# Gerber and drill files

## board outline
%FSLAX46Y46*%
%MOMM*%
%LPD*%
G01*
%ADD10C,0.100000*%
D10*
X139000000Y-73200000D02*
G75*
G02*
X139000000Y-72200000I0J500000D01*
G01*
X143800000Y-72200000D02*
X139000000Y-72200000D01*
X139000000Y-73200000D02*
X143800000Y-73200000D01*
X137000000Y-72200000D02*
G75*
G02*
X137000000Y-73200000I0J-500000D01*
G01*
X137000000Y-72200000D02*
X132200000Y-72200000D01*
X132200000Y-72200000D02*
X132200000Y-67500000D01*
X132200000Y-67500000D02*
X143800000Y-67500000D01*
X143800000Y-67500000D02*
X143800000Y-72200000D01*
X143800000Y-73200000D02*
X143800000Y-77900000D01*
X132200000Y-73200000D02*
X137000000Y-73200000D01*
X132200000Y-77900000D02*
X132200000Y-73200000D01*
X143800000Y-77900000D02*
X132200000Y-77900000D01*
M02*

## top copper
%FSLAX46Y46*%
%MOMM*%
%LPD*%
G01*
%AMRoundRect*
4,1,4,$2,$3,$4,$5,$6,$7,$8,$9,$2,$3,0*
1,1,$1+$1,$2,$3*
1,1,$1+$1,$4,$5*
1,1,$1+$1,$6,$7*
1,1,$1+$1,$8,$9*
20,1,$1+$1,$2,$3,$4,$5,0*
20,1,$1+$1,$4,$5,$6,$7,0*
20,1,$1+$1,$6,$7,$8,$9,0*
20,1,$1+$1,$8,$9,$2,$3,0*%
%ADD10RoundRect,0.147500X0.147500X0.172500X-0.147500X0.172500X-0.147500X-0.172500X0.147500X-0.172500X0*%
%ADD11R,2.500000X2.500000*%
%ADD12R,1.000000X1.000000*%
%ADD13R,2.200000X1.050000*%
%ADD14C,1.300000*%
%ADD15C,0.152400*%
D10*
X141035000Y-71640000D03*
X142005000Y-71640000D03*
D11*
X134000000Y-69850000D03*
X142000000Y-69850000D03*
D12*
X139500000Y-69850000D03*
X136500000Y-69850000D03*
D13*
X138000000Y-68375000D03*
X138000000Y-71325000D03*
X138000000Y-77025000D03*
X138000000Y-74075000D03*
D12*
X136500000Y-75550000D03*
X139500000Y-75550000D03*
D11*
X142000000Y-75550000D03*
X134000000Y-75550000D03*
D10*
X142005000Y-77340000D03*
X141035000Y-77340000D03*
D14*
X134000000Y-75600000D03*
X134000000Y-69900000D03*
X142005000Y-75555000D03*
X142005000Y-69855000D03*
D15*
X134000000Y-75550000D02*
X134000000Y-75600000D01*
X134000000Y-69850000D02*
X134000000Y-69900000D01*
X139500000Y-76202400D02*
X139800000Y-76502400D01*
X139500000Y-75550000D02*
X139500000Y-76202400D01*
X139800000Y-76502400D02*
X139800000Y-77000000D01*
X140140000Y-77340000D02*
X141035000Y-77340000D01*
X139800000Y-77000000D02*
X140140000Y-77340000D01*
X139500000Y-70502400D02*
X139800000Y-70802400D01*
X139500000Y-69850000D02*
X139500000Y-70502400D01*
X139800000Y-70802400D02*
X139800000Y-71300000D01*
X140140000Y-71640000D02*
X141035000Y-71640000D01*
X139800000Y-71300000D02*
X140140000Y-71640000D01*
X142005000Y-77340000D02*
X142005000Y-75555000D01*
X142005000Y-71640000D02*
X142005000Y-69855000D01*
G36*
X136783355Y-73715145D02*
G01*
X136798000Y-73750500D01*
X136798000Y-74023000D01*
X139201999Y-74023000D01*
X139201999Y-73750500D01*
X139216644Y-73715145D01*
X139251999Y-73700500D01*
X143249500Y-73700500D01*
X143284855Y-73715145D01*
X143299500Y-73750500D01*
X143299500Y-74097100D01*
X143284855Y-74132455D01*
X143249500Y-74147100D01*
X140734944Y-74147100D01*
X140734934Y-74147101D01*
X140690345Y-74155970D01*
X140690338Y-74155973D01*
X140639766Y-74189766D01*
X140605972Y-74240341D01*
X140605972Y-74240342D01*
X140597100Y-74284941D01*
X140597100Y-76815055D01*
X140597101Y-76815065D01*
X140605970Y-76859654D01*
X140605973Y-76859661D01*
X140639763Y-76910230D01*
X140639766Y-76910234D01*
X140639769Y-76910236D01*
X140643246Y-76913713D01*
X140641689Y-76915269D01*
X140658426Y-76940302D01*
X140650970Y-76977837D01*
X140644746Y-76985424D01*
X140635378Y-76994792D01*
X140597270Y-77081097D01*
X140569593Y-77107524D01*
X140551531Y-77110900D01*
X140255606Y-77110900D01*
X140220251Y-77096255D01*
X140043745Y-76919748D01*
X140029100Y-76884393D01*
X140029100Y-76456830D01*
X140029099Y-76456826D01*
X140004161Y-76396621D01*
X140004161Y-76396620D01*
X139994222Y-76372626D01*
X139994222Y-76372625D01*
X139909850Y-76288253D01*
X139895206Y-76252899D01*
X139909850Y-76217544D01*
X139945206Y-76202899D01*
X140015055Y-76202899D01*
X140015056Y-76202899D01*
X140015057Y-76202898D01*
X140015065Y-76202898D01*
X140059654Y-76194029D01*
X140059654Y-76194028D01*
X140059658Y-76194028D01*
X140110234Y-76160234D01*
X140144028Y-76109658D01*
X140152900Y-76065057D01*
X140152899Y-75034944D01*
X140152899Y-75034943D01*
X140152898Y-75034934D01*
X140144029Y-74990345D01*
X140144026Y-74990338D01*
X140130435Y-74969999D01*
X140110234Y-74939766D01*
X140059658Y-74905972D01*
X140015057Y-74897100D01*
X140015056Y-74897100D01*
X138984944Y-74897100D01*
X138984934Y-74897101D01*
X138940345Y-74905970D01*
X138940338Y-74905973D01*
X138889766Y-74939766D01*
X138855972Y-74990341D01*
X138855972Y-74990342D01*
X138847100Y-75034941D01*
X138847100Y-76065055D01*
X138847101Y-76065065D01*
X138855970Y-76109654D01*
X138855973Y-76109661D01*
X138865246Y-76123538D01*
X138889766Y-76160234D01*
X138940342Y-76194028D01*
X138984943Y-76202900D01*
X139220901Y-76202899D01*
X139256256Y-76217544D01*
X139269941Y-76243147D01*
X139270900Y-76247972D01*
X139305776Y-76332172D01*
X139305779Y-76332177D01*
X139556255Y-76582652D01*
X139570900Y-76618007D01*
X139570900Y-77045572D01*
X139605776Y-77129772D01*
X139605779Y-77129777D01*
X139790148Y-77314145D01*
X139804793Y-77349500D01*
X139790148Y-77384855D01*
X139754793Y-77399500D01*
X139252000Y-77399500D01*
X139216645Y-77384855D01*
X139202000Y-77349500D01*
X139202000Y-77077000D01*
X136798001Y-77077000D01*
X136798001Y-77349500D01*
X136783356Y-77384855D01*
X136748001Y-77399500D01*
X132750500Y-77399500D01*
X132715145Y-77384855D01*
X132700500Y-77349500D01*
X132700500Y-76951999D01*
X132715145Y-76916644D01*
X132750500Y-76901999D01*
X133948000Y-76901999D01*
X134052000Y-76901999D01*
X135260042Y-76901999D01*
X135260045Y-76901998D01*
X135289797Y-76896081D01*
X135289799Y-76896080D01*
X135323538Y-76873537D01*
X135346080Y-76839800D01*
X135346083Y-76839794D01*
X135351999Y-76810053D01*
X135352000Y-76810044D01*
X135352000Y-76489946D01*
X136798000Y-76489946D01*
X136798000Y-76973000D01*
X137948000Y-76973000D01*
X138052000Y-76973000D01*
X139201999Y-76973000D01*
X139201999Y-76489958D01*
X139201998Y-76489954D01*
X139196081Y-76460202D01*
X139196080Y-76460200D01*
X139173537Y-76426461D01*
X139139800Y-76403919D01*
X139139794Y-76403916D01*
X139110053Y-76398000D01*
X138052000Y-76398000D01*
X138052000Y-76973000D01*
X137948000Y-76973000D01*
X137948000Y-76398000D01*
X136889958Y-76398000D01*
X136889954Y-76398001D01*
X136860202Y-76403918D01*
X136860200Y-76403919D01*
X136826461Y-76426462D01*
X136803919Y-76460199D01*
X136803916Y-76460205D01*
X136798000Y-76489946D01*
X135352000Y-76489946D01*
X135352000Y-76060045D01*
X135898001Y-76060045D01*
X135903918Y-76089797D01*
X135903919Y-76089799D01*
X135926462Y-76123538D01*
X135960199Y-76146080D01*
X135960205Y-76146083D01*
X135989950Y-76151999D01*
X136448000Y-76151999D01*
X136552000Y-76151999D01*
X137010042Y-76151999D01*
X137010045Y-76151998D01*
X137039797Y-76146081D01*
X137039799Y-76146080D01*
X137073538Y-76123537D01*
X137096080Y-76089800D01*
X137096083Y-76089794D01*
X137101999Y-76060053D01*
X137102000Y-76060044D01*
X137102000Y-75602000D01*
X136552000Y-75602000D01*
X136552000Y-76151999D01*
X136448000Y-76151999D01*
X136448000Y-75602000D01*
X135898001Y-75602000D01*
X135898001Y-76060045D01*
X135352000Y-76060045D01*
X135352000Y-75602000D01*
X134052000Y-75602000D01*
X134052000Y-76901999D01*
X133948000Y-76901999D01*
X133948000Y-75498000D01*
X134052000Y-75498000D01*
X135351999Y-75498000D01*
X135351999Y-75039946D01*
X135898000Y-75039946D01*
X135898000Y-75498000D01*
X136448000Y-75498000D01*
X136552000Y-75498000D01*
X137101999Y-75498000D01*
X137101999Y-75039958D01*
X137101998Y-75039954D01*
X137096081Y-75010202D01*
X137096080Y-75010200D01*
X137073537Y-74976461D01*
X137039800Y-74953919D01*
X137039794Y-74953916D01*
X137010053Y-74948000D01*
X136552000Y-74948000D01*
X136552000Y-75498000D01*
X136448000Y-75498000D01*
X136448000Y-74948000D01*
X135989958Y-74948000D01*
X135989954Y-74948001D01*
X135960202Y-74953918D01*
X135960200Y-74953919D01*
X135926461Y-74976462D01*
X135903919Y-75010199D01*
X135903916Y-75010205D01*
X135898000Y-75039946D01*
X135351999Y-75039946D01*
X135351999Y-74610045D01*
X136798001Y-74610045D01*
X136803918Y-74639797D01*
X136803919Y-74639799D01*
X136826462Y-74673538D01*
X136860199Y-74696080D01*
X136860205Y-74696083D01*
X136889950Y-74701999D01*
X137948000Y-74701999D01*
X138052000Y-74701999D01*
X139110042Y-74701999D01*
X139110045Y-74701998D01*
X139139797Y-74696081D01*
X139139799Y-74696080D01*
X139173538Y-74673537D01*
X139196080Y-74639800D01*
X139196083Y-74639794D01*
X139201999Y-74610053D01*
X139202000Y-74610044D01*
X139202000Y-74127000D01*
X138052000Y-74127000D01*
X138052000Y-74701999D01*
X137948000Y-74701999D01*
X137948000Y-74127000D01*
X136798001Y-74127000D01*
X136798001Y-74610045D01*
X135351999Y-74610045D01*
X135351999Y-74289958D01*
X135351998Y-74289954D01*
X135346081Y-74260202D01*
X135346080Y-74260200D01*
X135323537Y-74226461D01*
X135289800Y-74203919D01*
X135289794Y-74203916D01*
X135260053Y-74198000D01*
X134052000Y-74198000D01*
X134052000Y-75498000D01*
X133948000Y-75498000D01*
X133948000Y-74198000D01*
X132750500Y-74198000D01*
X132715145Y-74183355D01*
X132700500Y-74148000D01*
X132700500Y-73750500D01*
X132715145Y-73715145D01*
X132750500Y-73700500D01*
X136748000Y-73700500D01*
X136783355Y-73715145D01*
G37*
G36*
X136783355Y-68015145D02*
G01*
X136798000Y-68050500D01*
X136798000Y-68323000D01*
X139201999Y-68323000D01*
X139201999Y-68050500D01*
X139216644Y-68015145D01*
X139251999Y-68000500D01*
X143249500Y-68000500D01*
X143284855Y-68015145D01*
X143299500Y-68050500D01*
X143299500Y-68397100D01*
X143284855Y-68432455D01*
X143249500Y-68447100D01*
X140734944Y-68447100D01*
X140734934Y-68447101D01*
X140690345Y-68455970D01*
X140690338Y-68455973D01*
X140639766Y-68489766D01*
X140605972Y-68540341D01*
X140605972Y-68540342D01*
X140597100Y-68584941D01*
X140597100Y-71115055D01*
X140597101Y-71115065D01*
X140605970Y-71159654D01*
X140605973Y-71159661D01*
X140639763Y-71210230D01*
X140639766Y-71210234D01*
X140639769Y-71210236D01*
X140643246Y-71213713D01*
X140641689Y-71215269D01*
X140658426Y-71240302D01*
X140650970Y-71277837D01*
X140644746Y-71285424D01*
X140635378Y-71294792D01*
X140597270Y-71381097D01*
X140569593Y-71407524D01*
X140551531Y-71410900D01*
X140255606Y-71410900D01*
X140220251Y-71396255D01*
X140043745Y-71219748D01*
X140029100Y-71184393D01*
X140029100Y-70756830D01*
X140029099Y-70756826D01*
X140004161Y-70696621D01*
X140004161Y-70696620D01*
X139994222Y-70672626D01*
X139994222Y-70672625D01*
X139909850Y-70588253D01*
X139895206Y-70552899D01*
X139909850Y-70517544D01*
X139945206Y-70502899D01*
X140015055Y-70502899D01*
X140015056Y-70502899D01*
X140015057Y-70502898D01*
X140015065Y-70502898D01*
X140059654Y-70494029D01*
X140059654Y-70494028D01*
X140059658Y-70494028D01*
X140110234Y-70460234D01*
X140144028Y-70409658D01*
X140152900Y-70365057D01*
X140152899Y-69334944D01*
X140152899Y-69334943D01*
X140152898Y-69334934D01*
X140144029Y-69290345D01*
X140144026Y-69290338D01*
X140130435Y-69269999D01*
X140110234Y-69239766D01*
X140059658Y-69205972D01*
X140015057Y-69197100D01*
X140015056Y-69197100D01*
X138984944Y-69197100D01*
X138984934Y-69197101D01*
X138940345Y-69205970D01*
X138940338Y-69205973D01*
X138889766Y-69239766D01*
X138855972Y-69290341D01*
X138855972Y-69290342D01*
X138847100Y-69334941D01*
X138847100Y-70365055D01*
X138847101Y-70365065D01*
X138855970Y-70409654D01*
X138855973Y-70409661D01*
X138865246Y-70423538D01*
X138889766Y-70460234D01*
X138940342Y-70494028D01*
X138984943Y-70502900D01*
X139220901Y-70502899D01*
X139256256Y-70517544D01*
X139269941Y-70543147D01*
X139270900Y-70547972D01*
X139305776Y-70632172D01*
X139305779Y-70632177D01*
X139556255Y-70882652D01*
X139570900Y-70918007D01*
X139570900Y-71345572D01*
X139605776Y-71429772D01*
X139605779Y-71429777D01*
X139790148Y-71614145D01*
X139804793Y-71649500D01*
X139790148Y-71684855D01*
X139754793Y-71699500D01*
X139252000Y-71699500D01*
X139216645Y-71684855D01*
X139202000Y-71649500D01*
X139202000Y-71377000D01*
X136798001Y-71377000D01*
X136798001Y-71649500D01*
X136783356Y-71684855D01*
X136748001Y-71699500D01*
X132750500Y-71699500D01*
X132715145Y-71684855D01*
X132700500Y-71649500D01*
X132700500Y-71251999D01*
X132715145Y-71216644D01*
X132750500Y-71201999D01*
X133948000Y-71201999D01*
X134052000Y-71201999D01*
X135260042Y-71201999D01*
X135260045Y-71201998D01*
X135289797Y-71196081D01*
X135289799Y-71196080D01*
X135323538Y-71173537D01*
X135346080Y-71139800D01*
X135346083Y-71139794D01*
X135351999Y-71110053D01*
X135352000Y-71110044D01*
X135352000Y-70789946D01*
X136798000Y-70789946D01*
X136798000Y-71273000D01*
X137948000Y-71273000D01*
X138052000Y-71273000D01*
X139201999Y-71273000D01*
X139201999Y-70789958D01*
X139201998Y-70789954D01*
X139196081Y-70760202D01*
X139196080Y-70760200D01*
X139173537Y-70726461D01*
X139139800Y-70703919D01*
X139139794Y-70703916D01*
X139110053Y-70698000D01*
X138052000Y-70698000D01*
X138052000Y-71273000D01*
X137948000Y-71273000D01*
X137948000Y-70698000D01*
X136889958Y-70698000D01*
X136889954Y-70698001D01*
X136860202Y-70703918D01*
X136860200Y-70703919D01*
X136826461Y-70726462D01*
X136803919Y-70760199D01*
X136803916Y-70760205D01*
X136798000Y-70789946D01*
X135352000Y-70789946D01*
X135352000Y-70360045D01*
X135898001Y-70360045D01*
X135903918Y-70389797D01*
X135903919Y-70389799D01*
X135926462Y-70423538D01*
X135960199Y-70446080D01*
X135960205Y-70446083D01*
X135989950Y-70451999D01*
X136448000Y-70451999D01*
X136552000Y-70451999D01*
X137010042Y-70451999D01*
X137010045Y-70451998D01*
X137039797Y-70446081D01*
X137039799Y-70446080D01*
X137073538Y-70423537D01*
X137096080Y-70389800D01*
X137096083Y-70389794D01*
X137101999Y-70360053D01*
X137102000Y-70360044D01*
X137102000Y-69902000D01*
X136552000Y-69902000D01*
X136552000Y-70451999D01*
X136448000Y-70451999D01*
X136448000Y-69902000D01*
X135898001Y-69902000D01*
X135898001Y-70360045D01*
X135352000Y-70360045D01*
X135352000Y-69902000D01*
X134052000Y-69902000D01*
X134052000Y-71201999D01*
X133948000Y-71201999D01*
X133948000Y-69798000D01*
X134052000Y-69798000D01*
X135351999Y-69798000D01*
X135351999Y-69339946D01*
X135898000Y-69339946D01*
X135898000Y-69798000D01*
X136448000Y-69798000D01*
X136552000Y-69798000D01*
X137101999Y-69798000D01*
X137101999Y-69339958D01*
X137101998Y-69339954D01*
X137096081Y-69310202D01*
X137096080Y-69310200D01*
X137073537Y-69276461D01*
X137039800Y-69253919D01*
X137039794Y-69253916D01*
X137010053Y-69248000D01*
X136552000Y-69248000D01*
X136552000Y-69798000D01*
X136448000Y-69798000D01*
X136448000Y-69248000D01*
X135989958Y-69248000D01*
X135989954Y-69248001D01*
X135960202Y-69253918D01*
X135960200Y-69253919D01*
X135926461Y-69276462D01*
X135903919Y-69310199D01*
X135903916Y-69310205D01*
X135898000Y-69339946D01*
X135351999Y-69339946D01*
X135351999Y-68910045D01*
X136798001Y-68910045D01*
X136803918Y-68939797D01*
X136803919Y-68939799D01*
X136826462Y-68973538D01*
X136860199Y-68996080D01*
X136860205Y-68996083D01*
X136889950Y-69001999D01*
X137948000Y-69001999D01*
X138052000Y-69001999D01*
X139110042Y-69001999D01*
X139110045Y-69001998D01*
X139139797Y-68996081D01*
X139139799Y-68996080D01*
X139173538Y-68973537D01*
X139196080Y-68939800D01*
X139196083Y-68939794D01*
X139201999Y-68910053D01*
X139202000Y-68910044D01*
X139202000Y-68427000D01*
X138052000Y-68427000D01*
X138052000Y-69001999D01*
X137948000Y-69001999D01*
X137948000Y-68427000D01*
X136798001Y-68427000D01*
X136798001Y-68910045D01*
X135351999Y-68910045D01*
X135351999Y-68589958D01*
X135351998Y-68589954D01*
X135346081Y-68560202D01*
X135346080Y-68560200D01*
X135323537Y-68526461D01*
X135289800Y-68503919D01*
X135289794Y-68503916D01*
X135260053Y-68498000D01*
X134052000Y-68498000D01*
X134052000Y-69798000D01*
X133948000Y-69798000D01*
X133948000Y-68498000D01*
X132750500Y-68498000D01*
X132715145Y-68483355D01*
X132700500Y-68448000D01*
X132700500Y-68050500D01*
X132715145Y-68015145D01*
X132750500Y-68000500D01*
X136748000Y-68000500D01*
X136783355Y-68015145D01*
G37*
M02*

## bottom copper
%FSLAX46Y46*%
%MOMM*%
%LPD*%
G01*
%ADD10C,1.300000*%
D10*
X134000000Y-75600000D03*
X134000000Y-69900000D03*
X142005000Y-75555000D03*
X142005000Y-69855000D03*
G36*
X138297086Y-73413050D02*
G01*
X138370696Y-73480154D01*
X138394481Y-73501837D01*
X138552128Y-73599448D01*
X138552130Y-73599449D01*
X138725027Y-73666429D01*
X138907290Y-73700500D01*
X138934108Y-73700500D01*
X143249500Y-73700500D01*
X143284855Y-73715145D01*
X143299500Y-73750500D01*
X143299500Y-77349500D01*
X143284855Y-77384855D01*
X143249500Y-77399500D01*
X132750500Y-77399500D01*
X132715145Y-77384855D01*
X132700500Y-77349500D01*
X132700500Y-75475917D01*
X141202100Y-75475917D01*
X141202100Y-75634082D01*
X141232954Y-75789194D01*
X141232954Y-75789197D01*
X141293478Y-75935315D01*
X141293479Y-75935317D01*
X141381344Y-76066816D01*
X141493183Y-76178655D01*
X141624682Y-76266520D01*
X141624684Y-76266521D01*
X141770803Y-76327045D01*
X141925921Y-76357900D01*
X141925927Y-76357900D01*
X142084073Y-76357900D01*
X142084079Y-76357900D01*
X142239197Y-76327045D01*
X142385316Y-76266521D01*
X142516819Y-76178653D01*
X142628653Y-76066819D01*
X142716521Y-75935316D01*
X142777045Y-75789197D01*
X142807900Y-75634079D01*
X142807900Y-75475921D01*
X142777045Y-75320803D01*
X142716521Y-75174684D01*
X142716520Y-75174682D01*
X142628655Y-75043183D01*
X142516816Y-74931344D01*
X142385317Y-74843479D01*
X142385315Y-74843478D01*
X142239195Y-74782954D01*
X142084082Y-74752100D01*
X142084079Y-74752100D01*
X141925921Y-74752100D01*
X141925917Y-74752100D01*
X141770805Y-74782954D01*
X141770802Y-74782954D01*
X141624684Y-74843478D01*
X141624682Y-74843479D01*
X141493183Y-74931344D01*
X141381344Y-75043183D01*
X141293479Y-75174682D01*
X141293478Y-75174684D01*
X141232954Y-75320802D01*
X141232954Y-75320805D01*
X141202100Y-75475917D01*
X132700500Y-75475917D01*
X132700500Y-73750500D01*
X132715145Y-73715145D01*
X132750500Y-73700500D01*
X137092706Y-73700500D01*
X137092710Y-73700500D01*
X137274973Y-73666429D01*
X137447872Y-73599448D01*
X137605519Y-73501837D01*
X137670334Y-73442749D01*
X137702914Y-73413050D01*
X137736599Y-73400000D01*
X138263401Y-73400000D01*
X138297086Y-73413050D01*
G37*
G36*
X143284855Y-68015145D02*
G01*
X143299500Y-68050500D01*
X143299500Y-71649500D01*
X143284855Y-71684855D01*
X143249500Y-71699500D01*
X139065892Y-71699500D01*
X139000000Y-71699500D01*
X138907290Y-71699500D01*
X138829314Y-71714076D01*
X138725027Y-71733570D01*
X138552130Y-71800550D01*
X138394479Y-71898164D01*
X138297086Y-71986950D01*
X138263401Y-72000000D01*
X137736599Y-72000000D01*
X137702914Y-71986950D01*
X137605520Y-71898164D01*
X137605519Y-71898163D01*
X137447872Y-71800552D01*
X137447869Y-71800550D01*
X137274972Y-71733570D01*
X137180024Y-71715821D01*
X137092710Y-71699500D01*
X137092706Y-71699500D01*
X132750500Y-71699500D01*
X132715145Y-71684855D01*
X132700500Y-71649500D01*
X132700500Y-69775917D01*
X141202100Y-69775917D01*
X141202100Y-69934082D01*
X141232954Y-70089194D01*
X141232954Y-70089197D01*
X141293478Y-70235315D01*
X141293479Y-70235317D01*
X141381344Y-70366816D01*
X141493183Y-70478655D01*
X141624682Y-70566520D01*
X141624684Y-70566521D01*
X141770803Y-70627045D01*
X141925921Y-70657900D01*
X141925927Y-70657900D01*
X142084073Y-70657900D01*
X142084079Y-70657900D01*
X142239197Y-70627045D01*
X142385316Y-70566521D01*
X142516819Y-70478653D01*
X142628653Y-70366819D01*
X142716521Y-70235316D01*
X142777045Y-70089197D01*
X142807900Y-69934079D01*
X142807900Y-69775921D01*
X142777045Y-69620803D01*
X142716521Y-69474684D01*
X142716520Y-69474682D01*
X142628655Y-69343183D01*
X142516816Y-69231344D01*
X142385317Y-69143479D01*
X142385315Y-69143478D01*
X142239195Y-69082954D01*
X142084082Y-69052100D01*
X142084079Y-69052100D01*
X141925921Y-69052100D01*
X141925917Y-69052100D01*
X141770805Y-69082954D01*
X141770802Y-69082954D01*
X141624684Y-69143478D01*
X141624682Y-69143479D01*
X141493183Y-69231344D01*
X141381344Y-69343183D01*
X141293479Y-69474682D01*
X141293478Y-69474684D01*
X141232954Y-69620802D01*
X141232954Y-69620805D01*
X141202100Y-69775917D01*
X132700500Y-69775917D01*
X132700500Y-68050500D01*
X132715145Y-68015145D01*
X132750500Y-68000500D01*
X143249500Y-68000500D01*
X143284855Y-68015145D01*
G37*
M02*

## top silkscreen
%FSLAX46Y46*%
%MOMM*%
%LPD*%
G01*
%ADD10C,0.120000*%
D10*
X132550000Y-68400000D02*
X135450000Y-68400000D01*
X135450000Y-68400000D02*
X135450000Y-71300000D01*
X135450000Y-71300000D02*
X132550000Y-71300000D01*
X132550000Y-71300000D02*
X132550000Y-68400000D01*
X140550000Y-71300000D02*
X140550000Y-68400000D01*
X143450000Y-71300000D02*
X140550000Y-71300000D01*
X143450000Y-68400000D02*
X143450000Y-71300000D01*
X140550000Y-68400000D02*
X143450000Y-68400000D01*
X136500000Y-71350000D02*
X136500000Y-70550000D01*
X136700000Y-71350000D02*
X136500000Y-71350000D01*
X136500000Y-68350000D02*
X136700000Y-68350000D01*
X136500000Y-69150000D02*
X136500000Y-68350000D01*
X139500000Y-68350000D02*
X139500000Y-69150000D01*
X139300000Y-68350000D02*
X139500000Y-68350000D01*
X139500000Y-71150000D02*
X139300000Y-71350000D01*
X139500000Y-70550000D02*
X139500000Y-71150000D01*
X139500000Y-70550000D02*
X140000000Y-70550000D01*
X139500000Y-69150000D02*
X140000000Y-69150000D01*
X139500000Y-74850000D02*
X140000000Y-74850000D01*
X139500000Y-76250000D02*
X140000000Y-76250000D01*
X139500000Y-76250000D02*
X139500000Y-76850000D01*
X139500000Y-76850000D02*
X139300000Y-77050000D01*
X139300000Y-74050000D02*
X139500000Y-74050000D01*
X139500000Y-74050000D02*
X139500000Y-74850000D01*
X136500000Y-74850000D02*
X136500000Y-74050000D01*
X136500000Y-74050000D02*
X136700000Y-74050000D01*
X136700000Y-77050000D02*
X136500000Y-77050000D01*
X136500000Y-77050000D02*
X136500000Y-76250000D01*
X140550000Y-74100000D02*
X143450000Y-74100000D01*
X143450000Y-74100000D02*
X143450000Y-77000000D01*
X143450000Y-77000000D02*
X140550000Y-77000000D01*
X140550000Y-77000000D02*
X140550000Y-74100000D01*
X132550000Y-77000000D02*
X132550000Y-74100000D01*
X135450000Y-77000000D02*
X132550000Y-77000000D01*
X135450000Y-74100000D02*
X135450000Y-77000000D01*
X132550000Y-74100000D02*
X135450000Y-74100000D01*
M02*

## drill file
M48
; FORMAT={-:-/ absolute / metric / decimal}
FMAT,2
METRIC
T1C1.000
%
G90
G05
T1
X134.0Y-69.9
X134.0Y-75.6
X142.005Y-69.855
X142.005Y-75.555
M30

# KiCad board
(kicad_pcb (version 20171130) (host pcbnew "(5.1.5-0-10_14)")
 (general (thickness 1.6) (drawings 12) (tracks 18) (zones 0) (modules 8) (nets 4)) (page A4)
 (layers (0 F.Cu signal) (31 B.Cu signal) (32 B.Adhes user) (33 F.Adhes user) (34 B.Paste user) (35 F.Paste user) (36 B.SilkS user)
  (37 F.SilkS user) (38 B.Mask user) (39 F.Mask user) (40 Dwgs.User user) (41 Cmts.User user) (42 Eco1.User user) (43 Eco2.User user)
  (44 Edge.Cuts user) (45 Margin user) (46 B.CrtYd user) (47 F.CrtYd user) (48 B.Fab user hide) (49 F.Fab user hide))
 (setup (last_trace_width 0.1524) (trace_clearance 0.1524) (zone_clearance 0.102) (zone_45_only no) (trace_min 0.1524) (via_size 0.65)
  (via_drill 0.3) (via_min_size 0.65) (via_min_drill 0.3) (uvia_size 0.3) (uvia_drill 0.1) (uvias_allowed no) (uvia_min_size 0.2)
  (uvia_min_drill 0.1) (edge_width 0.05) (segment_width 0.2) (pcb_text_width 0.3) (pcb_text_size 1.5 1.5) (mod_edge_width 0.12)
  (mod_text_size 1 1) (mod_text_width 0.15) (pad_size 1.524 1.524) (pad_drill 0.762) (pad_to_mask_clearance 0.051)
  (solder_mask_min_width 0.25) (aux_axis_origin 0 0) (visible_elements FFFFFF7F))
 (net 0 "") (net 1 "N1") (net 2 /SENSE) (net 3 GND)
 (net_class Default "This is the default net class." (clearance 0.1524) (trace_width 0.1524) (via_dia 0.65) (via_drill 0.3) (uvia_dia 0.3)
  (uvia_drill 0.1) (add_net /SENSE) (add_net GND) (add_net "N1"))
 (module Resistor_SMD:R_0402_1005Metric (layer F.Cu) (at 141.52 71.64 180)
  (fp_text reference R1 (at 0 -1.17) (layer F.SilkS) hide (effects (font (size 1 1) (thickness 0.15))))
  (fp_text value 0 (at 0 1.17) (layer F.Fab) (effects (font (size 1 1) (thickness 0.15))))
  (pad 2 smd roundrect (at 0.485 0 180) (size 0.59 0.64) (layers F.Cu F.Paste F.Mask) (roundrect_rratio 0.25) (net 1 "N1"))
  (pad 1 smd roundrect (at -0.485 0 180) (size 0.59 0.64) (layers F.Cu F.Paste F.Mask) (roundrect_rratio 0.25) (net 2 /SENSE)))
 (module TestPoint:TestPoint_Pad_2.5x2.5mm (layer F.Cu) (at 134 69.85)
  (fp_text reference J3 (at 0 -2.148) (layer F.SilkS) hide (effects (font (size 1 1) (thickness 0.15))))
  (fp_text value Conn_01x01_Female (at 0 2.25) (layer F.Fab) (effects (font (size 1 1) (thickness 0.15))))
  (fp_line (start -1.45 -1.45) (end 1.45 -1.45) (layer F.SilkS) (width 0.12))
  (fp_line (start 1.45 -1.45) (end 1.45 1.45) (layer F.SilkS) (width 0.12))
  (fp_line (start 1.45 1.45) (end -1.45 1.45) (layer F.SilkS) (width 0.12))
  (fp_line (start -1.45 1.45) (end -1.45 -1.45) (layer F.SilkS) (width 0.12))
  (pad 1 smd rect (at 0 0) (size 2.5 2.5) (layers F.Cu F.Mask) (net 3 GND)))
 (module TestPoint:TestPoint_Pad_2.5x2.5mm (layer F.Cu) (at 142 69.85)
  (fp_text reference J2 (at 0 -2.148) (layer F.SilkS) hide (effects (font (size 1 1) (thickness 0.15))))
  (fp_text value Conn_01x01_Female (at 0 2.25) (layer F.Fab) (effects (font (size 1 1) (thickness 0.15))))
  (fp_line (start -1.45 1.45) (end -1.45 -1.45) (layer F.SilkS) (width 0.12))
  (fp_line (start 1.45 1.45) (end -1.45 1.45) (layer F.SilkS) (width 0.12))
  (fp_line (start 1.45 -1.45) (end 1.45 1.45) (layer F.SilkS) (width 0.12))
  (fp_line (start -1.45 -1.45) (end 1.45 -1.45) (layer F.SilkS) (width 0.12))
  (pad 1 smd rect (at 0 0) (size 2.5 2.5) (layers F.Cu F.Mask) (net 2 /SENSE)))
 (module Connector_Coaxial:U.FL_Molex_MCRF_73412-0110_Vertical (layer F.Cu) (at 138 69.85 90)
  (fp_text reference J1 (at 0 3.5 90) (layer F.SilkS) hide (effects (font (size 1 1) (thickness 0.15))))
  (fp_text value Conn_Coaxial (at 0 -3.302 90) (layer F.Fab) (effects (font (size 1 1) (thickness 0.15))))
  (fp_line (start -1.5 -1.5) (end -0.7 -1.5) (layer F.SilkS) (width 0.12))
  (fp_line (start -1.5 -1.3) (end -1.5 -1.5) (layer F.SilkS) (width 0.12))
  (fp_line (start 1.5 -1.5) (end 1.5 -1.3) (layer F.SilkS) (width 0.12))
  (fp_line (start 0.7 -1.5) (end 1.5 -1.5) (layer F.SilkS) (width 0.12))
  (fp_line (start 1.5 1.5) (end 0.7 1.5) (layer F.SilkS) (width 0.12))
  (fp_line (start 1.5 1.3) (end 1.5 1.5) (layer F.SilkS) (width 0.12))
  (fp_line (start -1.3 1.5) (end -1.5 1.3) (layer F.SilkS) (width 0.12))
  (fp_line (start -0.7 1.5) (end -1.3 1.5) (layer F.SilkS) (width 0.12))
  (fp_line (start -0.7 1.5) (end -0.7 2) (layer F.SilkS) (width 0.12))
  (fp_line (start 0.7 1.5) (end 0.7 2) (layer F.SilkS) (width 0.12))
  (pad 1 smd rect (at 0 1.5 90) (size 1 1) (layers F.Cu F.Paste F.Mask) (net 1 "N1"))
  (pad 2 smd rect (at 0 -1.5 90) (size 1 1) (layers F.Cu F.Paste F.Mask) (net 3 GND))
  (pad 2 smd rect (at 1.475 0 90) (size 1.05 2.2) (layers F.Cu F.Paste F.Mask) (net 3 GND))
  (pad 2 smd rect (at -1.475 0 90) (size 1.05 2.2) (layers F.Cu F.Paste F.Mask) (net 3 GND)))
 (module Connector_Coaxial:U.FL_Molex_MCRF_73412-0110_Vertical (layer F.Cu) (at 138 75.55 90)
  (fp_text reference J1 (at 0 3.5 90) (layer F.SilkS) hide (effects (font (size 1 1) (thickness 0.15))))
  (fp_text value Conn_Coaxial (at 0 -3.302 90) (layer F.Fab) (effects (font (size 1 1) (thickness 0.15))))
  (fp_line (start 0.7 1.5) (end 0.7 2) (layer F.SilkS) (width 0.12))
  (fp_line (start -0.7 1.5) (end -0.7 2) (layer F.SilkS) (width 0.12))
  (fp_line (start -0.7 1.5) (end -1.3 1.5) (layer F.SilkS) (width 0.12))
  (fp_line (start -1.3 1.5) (end -1.5 1.3) (layer F.SilkS) (width 0.12))
  (fp_line (start 1.5 1.3) (end 1.5 1.5) (layer F.SilkS) (width 0.12))
  (fp_line (start 1.5 1.5) (end 0.7 1.5) (layer F.SilkS) (width 0.12))
  (fp_line (start 0.7 -1.5) (end 1.5 -1.5) (layer F.SilkS) (width 0.12))
  (fp_line (start 1.5 -1.5) (end 1.5 -1.3) (layer F.SilkS) (width 0.12))
  (fp_line (start -1.5 -1.3) (end -1.5 -1.5) (layer F.SilkS) (width 0.12))
  (fp_line (start -1.5 -1.5) (end -0.7 -1.5) (layer F.SilkS) (width 0.12))
  (pad 2 smd rect (at -1.475 0 90) (size 1.05 2.2) (layers F.Cu F.Paste F.Mask) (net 3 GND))
  (pad 2 smd rect (at 1.475 0 90) (size 1.05 2.2) (layers F.Cu F.Paste F.Mask) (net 3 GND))
  (pad 2 smd rect (at 0 -1.5 90) (size 1 1) (layers F.Cu F.Paste F.Mask) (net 3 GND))
  (pad 1 smd rect (at 0 1.5 90) (size 1 1) (layers F.Cu F.Paste F.Mask) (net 1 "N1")))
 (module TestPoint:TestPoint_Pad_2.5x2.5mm (layer F.Cu) (at 142 75.55)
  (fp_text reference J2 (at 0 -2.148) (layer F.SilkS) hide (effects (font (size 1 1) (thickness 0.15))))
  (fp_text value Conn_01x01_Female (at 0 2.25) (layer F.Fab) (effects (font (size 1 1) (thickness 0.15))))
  (fp_line (start -1.45 -1.45) (end 1.45 -1.45) (layer F.SilkS) (width 0.12))
  (fp_line (start 1.45 -1.45) (end 1.45 1.45) (layer F.SilkS) (width 0.12))
  (fp_line (start 1.45 1.45) (end -1.45 1.45) (layer F.SilkS) (width 0.12))
  (fp_line (start -1.45 1.45) (end -1.45 -1.45) (layer F.SilkS) (width 0.12))
  (pad 1 smd rect (at 0 0) (size 2.5 2.5) (layers F.Cu F.Mask) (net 2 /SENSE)))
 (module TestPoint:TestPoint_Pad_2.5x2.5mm (layer F.Cu) (at 134 75.55)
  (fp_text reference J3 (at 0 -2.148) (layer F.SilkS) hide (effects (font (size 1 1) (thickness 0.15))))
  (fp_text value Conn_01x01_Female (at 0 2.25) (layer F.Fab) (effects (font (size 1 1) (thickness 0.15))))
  (fp_line (start -1.45 1.45) (end -1.45 -1.45) (layer F.SilkS) (width 0.12))
  (fp_line (start 1.45 1.45) (end -1.45 1.45) (layer F.SilkS) (width 0.12))
  (fp_line (start 1.45 -1.45) (end 1.45 1.45) (layer F.SilkS) (width 0.12))
  (fp_line (start -1.45 -1.45) (end 1.45 -1.45) (layer F.SilkS) (width 0.12))
  (pad 1 smd rect (at 0 0) (size 2.5 2.5) (layers F.Cu F.Mask) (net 3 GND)))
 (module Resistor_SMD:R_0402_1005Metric (layer F.Cu) (at 141.52 77.34 180)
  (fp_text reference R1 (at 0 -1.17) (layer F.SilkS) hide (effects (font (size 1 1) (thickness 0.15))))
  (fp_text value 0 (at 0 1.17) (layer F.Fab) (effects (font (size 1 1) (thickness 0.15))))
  (pad 1 smd roundrect (at -0.485 0 180) (size 0.59 0.64) (layers F.Cu F.Paste F.Mask) (roundrect_rratio 0.25) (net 2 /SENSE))
  (pad 2 smd roundrect (at 0.485 0 180) (size 0.59 0.64) (layers F.Cu F.Paste F.Mask) (roundrect_rratio 0.25) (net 1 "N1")))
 (gr_arc (start 139 72.7) (end 139 72.2) (angle -180) (layer Edge.Cuts) (width 0.1))
 (gr_line (start 143.8 72.2) (end 139 72.2) (layer Edge.Cuts) (width 0.1))
 (gr_line (start 139 73.2) (end 143.8 73.2) (layer Edge.Cuts) (width 0.1))
 (gr_arc (start 137 72.7) (end 137 73.2) (angle -180) (layer Edge.Cuts) (width 0.1))
 (gr_line (start 137 72.2) (end 132.2 72.2) (layer Edge.Cuts) (width 0.1))
 (gr_line (start 132.2 72.2) (end 132.2 67.5) (layer Edge.Cuts) (width 0.1))
 (gr_line (start 132.2 67.5) (end 143.8 67.5) (layer Edge.Cuts) (width 0.1))
 (gr_line (start 143.8 67.5) (end 143.8 72.2) (layer Edge.Cuts) (width 0.1))
 (gr_line (start 143.8 73.2) (end 143.8 77.9) (layer Edge.Cuts) (width 0.1))
 (gr_line (start 132.2 73.2) (end 137 73.2) (layer Edge.Cuts) (width 0.1))
 (gr_line (start 132.2 77.9) (end 132.2 73.2) (layer Edge.Cuts) (width 0.1))
 (gr_line (start 143.8 77.9) (end 132.2 77.9) (layer Edge.Cuts) (width 0.1))
 (via (at 134 75.6) (size 1.3) (drill 1) (layers F.Cu B.Cu) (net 3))
 (segment (start 134 75.55) (end 134 75.6) (width 0.1524) (layer F.Cu) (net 3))
 (via (at 134 69.9) (size 1.3) (drill 1) (layers F.Cu B.Cu) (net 3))
 (segment (start 134 69.85) (end 134 69.9) (width 0.1524) (layer F.Cu) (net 3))
 (segment (start 139.5 76.2024) (end 139.8 76.5024) (width 0.1524) (layer F.Cu) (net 1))
 (segment (start 139.5 75.55) (end 139.5 76.2024) (width 0.1524) (layer F.Cu) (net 1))
 (segment (start 139.8 76.5024) (end 139.8 77) (width 0.1524) (layer F.Cu) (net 1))
 (segment (start 140.14 77.34) (end 141.035 77.34) (width 0.1524) (layer F.Cu) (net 1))
 (segment (start 139.8 77) (end 140.14 77.34) (width 0.1524) (layer F.Cu) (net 1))
 (segment (start 139.5 70.5024) (end 139.8 70.8024) (width 0.1524) (layer F.Cu) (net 1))
 (segment (start 139.5 69.85) (end 139.5 70.5024) (width 0.1524) (layer F.Cu) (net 1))
 (segment (start 139.8 70.8024) (end 139.8 71.3) (width 0.1524) (layer F.Cu) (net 1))
 (segment (start 140.14 71.64) (end 141.035 71.64) (width 0.1524) (layer F.Cu) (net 1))
 (segment (start 139.8 71.3) (end 140.14 71.64) (width 0.1524) (layer F.Cu) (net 1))
 (segment (start 142.005 77.34) (end 142.005 75.555) (width 0.1524) (layer F.Cu) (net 2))
 (via (at 142.005 75.555) (size 1.3) (drill 1) (layers F.Cu B.Cu) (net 2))
 (segment (start 142.005 71.64) (end 142.005 69.855) (width 0.1524) (layer F.Cu) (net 2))
 (via (at 142.005 69.855) (size 1.3) (drill 1) (layers F.Cu B.Cu) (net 2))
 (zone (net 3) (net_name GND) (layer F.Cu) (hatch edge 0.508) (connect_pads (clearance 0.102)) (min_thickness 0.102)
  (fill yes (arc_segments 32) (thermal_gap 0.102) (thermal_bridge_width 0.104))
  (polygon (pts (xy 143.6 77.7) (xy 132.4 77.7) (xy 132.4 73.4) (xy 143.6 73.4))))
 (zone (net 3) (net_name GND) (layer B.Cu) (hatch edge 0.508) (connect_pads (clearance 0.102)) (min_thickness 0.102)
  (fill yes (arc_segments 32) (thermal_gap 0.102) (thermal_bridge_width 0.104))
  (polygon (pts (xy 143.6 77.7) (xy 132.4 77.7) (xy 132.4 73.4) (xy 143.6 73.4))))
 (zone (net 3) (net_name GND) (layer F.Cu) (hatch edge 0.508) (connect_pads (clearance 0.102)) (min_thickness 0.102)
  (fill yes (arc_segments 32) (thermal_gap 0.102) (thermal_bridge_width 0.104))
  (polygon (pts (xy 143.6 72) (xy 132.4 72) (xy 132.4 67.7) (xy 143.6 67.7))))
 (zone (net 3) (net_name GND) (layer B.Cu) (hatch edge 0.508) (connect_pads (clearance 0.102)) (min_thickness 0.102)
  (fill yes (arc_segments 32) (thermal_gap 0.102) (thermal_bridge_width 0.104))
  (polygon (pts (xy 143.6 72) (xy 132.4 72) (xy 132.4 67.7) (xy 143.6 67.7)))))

